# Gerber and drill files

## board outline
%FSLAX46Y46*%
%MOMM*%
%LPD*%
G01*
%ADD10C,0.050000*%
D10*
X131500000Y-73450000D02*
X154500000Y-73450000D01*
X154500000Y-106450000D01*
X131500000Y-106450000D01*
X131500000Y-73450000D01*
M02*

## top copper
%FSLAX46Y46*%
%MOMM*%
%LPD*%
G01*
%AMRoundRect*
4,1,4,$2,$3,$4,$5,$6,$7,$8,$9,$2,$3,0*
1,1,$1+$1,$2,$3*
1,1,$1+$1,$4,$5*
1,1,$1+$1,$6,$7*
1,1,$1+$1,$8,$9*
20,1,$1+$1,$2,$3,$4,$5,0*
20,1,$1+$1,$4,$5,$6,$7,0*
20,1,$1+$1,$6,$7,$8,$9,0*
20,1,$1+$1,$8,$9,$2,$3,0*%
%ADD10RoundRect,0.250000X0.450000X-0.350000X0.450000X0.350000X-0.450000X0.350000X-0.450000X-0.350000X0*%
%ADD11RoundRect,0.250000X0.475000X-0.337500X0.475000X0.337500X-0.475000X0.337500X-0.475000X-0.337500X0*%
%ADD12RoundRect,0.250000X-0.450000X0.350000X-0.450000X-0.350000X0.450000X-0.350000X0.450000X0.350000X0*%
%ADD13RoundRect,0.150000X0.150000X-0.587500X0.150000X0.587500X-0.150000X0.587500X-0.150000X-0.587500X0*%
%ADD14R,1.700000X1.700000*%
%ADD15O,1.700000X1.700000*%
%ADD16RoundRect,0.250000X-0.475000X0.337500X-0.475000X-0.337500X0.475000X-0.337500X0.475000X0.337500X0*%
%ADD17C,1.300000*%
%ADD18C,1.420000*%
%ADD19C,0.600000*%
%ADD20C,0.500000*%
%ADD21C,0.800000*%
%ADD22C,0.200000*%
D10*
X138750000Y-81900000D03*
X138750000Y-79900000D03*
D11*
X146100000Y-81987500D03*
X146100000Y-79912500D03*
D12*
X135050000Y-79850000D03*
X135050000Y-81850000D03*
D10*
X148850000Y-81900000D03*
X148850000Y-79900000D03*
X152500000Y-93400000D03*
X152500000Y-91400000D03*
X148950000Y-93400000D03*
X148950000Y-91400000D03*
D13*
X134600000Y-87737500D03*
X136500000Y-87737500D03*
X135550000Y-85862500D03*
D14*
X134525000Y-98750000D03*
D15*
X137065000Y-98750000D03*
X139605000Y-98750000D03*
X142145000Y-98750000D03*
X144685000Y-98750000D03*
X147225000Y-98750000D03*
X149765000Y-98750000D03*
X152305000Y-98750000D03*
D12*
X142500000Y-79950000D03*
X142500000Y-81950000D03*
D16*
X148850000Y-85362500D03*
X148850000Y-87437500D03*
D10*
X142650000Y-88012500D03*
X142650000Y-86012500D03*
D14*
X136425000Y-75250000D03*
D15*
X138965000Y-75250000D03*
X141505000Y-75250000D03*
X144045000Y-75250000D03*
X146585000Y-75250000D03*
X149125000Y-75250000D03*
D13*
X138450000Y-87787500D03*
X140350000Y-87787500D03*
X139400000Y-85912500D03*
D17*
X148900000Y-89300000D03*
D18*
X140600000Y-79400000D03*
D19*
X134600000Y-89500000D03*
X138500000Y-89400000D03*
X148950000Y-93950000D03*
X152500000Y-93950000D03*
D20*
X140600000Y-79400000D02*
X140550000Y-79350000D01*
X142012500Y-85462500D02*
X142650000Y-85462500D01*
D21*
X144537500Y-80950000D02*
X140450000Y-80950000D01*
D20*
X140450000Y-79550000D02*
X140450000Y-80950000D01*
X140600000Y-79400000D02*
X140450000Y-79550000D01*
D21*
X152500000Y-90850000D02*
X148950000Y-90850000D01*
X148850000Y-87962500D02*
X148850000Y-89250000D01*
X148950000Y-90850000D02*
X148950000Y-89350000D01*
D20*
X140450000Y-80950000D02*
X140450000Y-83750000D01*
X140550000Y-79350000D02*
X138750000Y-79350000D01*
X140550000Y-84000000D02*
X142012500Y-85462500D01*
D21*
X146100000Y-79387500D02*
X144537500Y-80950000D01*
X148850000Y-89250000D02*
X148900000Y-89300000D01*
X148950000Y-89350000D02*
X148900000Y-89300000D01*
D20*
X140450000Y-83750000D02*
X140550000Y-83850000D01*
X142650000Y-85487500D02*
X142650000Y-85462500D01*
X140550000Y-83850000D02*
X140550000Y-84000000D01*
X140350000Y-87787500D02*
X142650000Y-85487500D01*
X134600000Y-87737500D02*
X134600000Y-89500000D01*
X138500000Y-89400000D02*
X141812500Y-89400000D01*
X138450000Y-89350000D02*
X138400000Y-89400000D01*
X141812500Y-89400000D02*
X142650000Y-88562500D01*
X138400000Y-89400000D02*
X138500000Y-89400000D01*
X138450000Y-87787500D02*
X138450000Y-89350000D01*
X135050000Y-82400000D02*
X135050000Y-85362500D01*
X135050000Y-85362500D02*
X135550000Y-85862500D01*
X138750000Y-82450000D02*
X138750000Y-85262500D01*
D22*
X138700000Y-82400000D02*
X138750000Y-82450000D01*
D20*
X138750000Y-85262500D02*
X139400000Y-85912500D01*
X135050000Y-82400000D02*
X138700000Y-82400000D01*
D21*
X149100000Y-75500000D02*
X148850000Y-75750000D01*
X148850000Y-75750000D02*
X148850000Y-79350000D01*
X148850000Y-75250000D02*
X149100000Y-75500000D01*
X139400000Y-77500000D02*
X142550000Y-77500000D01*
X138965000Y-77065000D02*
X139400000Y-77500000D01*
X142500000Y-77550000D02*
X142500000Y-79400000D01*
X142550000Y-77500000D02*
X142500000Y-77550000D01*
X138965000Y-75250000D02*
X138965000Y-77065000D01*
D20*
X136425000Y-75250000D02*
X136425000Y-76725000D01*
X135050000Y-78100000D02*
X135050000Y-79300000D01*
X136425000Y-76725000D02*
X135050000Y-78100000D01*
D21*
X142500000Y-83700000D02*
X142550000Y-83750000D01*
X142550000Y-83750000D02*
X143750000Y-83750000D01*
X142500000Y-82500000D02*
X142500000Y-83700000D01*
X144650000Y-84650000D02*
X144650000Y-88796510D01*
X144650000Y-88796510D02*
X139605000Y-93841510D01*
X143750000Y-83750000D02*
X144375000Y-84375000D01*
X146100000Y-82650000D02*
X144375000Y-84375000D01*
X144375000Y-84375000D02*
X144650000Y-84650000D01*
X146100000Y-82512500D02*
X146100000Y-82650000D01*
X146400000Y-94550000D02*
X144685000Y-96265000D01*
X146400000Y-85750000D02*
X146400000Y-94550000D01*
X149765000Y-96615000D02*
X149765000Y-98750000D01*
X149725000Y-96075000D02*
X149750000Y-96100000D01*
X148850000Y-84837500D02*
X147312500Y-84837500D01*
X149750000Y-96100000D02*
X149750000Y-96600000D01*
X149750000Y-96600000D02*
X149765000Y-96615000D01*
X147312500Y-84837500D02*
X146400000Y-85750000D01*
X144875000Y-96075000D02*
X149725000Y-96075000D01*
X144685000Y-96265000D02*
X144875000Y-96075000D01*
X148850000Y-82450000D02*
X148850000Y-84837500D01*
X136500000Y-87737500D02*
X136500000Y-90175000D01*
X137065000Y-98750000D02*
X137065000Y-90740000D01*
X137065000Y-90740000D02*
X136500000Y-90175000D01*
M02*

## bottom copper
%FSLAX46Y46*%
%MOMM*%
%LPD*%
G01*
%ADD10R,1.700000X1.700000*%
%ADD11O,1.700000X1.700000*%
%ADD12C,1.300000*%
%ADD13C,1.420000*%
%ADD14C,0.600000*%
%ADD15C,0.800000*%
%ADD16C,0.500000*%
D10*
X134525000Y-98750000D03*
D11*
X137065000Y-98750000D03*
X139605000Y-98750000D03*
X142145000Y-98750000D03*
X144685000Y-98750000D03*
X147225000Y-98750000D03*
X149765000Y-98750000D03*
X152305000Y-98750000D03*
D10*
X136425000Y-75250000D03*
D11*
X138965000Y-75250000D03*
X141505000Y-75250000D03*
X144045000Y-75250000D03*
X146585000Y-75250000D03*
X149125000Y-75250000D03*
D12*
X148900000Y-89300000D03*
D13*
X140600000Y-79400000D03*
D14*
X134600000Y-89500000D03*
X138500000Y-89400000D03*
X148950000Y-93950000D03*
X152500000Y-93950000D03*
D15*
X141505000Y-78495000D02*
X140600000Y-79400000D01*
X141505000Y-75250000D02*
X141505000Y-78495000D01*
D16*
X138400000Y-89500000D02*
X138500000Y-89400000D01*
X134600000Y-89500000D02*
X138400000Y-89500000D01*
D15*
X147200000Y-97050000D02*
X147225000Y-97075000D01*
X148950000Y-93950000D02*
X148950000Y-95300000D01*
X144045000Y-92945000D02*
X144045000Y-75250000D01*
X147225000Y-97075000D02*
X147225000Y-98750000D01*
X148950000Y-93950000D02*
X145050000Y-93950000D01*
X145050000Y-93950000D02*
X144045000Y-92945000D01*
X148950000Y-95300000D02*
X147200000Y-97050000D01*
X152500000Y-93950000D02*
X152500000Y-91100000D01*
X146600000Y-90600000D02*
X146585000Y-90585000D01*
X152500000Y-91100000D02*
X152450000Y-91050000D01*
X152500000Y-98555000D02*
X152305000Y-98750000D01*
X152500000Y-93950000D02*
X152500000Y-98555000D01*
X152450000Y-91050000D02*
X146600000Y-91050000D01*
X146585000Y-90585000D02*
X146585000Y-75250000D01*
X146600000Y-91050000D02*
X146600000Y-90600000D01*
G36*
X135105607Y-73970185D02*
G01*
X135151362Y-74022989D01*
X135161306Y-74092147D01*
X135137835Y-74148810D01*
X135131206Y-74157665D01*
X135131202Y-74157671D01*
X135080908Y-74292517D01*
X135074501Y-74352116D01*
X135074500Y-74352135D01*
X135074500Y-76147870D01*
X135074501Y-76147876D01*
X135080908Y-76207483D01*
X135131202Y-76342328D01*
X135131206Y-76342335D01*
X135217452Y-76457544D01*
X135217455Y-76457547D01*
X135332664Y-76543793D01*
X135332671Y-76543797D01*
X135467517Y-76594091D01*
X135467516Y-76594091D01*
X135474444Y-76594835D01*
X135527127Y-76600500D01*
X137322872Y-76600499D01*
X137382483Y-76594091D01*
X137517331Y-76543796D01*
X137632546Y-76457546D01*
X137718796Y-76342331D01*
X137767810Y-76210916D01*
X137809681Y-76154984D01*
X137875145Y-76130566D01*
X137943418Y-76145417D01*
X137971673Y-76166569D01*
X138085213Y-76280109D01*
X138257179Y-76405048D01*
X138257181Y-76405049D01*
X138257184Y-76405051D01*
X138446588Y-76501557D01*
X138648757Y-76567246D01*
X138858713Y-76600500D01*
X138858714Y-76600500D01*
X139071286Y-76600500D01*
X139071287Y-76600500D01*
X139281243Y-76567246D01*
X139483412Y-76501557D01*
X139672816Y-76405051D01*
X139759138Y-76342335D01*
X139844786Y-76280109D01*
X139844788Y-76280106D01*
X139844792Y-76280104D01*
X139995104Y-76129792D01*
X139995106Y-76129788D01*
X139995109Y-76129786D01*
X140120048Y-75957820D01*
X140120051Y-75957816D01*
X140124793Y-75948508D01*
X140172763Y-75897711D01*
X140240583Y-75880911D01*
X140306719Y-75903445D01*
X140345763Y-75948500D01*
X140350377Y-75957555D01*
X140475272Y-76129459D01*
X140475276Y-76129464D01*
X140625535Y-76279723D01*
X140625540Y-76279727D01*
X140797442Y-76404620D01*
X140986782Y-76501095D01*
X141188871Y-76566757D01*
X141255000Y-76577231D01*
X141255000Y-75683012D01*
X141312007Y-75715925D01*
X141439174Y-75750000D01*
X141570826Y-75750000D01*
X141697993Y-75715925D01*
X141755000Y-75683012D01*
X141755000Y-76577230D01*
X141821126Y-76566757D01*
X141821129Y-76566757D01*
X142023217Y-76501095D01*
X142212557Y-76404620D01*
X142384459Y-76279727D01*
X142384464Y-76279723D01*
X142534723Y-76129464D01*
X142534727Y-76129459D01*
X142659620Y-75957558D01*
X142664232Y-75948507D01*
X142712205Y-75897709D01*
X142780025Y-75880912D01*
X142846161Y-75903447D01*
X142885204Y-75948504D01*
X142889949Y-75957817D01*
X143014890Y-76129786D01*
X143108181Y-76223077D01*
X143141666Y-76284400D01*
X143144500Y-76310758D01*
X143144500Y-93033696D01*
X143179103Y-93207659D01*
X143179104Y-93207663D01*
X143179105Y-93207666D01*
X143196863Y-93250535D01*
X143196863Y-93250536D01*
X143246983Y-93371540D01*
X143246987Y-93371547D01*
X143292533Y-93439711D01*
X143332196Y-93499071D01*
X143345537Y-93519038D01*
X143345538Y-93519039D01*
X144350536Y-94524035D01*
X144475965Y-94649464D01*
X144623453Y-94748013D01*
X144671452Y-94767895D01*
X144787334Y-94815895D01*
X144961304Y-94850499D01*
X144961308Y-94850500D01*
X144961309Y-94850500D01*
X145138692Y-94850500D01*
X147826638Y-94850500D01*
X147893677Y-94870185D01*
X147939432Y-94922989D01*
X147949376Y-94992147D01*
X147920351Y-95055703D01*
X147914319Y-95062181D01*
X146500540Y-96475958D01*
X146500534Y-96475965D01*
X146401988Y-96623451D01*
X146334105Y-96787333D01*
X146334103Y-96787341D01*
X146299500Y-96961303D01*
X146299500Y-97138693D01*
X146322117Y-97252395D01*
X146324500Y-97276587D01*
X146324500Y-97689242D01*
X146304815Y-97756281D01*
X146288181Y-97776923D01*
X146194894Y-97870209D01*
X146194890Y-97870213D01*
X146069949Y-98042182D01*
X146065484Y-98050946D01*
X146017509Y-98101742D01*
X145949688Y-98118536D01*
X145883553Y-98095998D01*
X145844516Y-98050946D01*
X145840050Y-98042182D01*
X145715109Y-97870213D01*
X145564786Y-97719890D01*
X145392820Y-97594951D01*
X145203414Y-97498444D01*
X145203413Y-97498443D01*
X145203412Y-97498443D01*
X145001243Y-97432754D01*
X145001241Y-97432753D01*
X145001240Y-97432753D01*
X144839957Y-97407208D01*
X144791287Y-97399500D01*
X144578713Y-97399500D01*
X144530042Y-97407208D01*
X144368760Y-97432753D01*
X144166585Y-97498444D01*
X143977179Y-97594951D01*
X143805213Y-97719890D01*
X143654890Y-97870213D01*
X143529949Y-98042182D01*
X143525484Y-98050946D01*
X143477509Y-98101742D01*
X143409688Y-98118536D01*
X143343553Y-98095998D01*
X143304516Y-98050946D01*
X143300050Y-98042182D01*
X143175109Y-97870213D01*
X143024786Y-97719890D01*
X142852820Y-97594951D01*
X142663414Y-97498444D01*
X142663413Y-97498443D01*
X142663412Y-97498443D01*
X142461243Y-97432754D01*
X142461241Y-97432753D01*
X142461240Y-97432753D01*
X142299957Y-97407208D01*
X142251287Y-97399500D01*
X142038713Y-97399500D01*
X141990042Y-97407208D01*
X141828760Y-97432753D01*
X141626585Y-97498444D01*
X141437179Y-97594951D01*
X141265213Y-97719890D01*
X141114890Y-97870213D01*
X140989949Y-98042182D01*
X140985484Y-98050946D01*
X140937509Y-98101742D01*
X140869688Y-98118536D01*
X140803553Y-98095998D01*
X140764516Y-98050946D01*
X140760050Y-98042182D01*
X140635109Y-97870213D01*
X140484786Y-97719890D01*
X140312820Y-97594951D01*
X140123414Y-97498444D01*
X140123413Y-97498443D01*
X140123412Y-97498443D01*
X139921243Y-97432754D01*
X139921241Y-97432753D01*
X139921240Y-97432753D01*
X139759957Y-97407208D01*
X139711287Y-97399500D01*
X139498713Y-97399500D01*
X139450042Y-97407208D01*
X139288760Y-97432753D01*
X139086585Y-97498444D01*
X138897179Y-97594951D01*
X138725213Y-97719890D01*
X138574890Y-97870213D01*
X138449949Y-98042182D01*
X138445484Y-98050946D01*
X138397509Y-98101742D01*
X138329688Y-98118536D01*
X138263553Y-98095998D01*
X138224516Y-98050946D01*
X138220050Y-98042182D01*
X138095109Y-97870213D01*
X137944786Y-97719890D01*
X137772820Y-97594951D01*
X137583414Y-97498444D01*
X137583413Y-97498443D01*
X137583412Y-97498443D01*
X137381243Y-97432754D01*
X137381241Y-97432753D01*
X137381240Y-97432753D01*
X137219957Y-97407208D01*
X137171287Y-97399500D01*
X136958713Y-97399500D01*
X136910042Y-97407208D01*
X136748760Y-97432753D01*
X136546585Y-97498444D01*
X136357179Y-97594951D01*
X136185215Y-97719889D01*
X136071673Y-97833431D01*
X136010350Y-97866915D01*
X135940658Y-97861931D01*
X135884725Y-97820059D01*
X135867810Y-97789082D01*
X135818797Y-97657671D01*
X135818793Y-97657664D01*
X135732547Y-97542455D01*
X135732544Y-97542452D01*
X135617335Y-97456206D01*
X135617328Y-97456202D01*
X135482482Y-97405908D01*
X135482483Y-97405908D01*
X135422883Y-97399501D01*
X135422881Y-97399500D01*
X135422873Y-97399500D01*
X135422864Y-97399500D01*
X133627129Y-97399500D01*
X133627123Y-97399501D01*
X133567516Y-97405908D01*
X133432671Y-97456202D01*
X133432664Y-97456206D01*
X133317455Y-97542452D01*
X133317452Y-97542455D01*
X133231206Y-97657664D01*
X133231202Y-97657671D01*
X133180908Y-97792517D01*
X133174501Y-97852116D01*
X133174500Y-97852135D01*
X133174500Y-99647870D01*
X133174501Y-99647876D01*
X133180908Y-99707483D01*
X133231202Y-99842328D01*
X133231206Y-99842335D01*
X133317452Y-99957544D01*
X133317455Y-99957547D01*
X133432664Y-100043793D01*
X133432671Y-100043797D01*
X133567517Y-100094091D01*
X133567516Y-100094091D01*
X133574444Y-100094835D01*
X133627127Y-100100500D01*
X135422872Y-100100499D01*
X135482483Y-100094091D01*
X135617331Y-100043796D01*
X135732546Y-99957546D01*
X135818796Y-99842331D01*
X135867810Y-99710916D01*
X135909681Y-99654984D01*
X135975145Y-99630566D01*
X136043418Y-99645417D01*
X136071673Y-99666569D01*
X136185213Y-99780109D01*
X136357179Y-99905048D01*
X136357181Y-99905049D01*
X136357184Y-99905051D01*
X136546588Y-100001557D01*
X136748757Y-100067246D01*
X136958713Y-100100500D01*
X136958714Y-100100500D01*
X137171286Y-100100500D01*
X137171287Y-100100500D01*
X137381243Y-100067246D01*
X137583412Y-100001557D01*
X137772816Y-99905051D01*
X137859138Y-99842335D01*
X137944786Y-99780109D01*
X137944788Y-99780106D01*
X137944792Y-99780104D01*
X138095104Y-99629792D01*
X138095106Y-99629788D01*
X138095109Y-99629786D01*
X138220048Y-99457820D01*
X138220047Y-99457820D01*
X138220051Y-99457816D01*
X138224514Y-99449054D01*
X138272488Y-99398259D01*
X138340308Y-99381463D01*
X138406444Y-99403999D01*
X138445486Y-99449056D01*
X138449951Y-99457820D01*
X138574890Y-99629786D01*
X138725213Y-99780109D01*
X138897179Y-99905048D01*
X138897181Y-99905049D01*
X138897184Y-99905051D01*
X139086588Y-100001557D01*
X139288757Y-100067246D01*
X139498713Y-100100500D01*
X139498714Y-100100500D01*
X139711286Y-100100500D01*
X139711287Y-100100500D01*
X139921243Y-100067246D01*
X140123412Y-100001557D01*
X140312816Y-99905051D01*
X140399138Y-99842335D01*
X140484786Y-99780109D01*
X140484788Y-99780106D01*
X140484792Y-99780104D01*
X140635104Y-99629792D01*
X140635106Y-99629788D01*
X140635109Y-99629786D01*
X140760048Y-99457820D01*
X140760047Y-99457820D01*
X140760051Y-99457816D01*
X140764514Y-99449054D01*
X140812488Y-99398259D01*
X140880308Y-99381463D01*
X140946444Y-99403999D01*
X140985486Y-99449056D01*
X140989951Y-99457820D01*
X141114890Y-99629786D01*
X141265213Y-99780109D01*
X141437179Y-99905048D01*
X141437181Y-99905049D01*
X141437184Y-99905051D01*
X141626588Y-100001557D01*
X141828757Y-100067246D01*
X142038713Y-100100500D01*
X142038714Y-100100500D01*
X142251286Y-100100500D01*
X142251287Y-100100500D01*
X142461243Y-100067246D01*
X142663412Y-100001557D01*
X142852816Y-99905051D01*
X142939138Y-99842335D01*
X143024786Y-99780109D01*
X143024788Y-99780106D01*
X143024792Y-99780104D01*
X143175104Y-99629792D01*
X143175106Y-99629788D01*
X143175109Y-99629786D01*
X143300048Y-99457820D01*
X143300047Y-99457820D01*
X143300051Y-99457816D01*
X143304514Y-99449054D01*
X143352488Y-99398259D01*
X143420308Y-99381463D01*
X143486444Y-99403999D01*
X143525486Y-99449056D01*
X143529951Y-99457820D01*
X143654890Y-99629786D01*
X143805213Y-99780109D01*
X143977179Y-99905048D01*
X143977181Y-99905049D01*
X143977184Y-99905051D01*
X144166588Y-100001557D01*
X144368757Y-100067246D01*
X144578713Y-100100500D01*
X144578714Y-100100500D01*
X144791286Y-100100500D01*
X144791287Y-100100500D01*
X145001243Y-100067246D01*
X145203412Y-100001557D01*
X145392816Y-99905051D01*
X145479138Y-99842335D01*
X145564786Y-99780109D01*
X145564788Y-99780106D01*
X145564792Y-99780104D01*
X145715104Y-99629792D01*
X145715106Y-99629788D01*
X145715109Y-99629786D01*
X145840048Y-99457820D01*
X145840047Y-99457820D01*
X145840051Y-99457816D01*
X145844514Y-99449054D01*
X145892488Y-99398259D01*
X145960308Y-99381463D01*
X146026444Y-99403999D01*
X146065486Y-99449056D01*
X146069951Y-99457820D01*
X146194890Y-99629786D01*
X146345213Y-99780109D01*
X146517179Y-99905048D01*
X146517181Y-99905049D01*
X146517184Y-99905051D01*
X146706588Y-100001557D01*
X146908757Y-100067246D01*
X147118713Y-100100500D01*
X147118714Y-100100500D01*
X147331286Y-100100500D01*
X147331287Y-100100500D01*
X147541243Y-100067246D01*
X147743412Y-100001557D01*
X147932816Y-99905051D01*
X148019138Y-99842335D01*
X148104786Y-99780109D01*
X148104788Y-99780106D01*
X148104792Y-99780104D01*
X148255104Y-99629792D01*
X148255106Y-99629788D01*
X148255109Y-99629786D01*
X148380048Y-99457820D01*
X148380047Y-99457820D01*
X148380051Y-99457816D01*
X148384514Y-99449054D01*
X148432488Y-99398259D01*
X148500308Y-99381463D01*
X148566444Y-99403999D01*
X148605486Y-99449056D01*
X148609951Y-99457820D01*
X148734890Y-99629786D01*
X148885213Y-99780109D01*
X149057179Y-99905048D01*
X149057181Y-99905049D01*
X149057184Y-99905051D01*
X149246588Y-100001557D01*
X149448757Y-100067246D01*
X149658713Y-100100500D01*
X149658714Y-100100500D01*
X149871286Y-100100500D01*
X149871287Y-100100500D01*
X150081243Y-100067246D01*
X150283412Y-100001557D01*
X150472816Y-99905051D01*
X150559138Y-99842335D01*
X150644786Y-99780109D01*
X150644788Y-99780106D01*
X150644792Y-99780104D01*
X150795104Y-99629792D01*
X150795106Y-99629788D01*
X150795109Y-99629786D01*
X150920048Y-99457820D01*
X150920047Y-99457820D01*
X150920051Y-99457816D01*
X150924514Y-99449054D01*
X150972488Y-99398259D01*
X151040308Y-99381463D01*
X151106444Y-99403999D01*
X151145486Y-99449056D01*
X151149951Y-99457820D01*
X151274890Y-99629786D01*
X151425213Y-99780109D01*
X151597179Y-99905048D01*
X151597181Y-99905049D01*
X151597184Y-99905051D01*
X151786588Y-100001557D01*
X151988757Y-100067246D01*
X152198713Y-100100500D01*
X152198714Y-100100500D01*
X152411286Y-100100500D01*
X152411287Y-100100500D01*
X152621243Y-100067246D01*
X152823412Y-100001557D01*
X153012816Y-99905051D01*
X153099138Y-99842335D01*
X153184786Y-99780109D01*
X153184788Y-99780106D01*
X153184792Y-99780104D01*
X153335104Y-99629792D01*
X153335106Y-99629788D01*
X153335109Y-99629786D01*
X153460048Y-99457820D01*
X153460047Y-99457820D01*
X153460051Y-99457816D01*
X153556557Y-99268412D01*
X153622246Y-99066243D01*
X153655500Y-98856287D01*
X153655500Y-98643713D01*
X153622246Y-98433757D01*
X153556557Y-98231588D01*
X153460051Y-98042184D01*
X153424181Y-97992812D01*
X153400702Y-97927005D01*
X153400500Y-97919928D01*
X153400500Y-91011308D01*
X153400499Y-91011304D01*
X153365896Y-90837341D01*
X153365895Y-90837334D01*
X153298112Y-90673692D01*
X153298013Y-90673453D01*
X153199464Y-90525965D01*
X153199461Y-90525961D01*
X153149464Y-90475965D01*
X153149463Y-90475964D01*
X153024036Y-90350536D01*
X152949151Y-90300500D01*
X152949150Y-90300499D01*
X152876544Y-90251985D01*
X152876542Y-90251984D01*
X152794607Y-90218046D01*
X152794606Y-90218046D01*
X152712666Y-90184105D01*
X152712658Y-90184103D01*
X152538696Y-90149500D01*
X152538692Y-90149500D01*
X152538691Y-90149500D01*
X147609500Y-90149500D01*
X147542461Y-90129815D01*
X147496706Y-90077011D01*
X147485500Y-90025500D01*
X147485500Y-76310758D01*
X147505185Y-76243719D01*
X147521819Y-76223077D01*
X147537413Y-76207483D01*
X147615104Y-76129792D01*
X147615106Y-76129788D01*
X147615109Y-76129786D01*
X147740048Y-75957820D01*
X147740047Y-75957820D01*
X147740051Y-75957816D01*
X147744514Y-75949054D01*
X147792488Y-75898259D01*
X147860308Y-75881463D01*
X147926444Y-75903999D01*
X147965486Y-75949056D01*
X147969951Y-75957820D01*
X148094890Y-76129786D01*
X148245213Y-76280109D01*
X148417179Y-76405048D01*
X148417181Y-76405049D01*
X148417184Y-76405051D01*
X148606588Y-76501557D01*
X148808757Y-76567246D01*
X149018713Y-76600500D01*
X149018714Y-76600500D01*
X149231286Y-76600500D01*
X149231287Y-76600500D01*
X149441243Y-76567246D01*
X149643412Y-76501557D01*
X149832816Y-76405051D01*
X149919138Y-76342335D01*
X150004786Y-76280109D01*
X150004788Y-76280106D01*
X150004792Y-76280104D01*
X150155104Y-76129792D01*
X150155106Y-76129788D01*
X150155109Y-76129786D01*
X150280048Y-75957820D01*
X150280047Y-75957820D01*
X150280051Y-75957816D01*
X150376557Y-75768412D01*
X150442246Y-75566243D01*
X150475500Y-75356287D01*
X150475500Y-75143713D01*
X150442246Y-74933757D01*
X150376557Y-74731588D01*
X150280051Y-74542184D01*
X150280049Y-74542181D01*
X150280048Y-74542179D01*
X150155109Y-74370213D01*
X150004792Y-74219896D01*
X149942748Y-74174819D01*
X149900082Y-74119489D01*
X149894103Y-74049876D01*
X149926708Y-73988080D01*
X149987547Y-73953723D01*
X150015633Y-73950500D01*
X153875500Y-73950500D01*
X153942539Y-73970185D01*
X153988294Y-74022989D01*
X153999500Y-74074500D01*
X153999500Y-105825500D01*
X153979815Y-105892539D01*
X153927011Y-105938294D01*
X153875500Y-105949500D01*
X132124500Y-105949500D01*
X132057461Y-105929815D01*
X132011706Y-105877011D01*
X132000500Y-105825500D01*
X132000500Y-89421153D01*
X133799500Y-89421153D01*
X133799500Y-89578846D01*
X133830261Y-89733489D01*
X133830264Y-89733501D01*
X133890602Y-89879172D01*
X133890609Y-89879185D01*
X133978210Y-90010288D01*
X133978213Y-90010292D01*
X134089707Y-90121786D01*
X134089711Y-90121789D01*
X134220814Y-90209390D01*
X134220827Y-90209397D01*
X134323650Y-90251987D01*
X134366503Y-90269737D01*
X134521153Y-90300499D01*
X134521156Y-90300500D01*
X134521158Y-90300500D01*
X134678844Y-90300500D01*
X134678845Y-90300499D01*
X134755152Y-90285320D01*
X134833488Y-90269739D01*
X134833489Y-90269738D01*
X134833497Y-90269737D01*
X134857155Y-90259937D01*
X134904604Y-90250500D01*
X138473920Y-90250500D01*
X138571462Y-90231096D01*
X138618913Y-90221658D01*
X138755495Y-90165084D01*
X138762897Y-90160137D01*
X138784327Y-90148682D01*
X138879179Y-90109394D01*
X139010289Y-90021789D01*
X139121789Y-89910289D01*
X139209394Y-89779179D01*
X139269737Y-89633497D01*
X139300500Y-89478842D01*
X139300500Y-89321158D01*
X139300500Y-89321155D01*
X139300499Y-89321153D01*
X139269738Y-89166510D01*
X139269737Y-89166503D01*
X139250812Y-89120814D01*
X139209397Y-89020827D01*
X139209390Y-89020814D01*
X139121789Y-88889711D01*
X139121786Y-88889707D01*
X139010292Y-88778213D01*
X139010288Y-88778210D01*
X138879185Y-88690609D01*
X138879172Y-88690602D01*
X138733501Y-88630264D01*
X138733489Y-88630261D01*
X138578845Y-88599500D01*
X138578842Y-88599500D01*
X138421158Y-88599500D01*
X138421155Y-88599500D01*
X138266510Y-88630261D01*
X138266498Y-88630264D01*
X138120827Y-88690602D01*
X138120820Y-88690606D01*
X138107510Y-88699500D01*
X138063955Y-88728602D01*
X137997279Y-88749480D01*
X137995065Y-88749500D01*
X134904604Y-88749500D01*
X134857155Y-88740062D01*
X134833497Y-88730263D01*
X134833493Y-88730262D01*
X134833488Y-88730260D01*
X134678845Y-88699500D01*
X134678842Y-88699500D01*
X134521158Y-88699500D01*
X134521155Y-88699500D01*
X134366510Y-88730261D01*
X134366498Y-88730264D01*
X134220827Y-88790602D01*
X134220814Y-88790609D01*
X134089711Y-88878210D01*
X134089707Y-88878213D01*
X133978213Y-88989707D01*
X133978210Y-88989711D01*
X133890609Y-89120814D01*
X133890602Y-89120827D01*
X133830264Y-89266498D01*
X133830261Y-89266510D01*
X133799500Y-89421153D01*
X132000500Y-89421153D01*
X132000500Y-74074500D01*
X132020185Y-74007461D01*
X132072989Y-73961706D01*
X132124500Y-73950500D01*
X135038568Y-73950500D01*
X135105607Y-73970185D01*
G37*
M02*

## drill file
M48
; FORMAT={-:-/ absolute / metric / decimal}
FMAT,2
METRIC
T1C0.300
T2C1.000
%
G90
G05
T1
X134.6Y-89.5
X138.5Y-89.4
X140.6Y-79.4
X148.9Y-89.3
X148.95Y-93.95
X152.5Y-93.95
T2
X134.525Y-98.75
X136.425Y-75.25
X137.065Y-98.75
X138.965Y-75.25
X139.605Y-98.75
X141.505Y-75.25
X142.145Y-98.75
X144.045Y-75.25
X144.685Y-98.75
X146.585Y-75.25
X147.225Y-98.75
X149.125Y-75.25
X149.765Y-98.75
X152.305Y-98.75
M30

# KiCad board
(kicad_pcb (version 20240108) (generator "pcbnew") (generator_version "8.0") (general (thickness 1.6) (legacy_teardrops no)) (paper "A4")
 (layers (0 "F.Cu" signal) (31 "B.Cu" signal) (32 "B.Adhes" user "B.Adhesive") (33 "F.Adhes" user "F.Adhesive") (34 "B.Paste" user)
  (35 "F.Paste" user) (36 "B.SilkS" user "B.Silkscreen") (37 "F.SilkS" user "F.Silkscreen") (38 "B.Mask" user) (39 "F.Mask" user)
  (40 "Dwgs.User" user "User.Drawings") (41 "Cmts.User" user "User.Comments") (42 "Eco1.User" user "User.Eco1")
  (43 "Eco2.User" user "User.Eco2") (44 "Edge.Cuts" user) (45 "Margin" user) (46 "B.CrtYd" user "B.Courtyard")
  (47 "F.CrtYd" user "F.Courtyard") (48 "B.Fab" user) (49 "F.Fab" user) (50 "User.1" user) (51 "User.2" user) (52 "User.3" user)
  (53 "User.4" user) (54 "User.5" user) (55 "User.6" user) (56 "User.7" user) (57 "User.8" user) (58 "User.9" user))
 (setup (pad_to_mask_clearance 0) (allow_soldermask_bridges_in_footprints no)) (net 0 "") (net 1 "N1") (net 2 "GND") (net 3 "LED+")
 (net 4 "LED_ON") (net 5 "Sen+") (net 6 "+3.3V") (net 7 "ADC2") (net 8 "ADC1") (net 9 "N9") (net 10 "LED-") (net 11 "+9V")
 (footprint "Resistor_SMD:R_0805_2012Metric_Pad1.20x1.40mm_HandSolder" (layer "F.Cu") (at 138.75 80.9 90)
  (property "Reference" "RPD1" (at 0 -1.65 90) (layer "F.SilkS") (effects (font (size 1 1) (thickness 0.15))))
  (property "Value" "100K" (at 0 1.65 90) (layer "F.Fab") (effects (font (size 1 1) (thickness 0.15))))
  (pad "1" smd roundrect (at -1 0 90) (size 1.2 1.4) (layers "F.Cu" "F.Paste" "F.Mask") (roundrect_rratio 0.208333) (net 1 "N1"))
  (pad "2" smd roundrect (at 1 0 90) (size 1.2 1.4) (layers "F.Cu" "F.Paste" "F.Mask") (roundrect_rratio 0.208333) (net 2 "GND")))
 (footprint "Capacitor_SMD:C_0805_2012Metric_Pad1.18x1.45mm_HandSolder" (layer "F.Cu") (at 146.1 80.95 90)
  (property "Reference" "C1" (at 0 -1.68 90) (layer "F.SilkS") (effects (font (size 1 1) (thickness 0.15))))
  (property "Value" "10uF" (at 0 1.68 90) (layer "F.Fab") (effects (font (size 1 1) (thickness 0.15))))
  (pad "1" smd roundrect (at -1.0375 0 90) (size 1.175 1.45) (layers "F.Cu" "F.Paste" "F.Mask") (roundrect_rratio 0.212766) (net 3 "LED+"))
  (pad "2" smd roundrect (at 1.0375 0 90) (size 1.175 1.45) (layers "F.Cu" "F.Paste" "F.Mask") (roundrect_rratio 0.212766) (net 2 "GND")))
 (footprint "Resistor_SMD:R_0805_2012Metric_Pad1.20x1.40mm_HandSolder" (layer "F.Cu") (at 135.05 80.85 -90)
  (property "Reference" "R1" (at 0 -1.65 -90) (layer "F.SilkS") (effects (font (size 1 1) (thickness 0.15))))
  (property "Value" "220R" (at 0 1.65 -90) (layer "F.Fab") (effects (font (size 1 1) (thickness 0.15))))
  (pad "1" smd roundrect (at -1 0 270) (size 1.2 1.4) (layers "F.Cu" "F.Paste" "F.Mask") (roundrect_rratio 0.208333) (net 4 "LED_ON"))
  (pad "2" smd roundrect (at 1 0 270) (size 1.2 1.4) (layers "F.Cu" "F.Paste" "F.Mask") (roundrect_rratio 0.208333) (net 1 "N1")))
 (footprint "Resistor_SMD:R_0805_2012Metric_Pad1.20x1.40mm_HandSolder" (layer "F.Cu") (at 148.85 80.9 90)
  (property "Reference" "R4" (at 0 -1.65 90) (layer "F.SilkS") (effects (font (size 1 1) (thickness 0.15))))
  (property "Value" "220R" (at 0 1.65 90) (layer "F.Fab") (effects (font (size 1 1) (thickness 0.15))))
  (pad "1" smd roundrect (at -1 0 90) (size 1.2 1.4) (layers "F.Cu" "F.Paste" "F.Mask") (roundrect_rratio 0.208333) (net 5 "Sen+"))
  (pad "2" smd roundrect (at 1 0 90) (size 1.2 1.4) (layers "F.Cu" "F.Paste" "F.Mask") (roundrect_rratio 0.208333) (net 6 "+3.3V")))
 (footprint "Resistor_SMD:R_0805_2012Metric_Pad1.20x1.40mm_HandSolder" (layer "F.Cu") (at 152.5 92.4 90)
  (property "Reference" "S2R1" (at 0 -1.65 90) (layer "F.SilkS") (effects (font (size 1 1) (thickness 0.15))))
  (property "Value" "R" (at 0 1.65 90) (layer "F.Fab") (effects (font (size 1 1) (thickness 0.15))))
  (pad "1" smd roundrect (at -1 0 90) (size 1.2 1.4) (layers "F.Cu" "F.Paste" "F.Mask") (roundrect_rratio 0.208333) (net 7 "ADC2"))
  (pad "2" smd roundrect (at 1 0 90) (size 1.2 1.4) (layers "F.Cu" "F.Paste" "F.Mask") (roundrect_rratio 0.208333) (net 2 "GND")))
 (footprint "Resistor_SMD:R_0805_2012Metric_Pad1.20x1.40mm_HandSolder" (layer "F.Cu") (at 148.95 92.4 90)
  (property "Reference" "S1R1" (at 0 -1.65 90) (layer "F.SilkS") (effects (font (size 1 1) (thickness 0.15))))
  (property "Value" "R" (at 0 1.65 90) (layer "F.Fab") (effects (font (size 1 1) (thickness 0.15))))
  (pad "1" smd roundrect (at -1 0 90) (size 1.2 1.4) (layers "F.Cu" "F.Paste" "F.Mask") (roundrect_rratio 0.208333) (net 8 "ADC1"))
  (pad "2" smd roundrect (at 1 0 90) (size 1.2 1.4) (layers "F.Cu" "F.Paste" "F.Mask") (roundrect_rratio 0.208333) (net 2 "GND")))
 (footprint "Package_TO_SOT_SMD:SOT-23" (layer "F.Cu") (at 135.55 86.8 90)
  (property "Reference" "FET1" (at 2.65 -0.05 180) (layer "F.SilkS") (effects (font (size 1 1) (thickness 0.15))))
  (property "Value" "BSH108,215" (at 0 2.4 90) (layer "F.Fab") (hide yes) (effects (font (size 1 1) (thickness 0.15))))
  (pad "1" smd roundrect (at -0.9375 -0.95 90) (size 1.475 0.6) (layers "F.Cu" "F.Paste" "F.Mask") (roundrect_rratio 0.25) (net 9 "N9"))
  (pad "2" smd roundrect (at -0.9375 0.95 90) (size 1.475 0.6) (layers "F.Cu" "F.Paste" "F.Mask") (roundrect_rratio 0.25) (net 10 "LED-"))
  (pad "3" smd roundrect (at 0.9375 0 90) (size 1.475 0.6) (layers "F.Cu" "F.Paste" "F.Mask") (roundrect_rratio 0.25) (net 1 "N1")))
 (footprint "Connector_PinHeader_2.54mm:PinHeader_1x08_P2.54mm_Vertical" (layer "F.Cu") (at 134.525 98.75 90)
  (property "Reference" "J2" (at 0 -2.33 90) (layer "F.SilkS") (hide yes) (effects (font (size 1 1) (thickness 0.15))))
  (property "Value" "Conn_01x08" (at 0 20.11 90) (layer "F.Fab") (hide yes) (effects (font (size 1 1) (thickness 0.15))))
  (pad "1" thru_hole rect (at 0 0 90) (size 1.7 1.7) (drill 1) (layers "*.Cu" "*.Mask") (remove_unused_layers no) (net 3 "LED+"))
  (pad "2" thru_hole oval (at 0 2.54 90) (size 1.7 1.7) (drill 1) (layers "*.Cu" "*.Mask") (remove_unused_layers no) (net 10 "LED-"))
  (pad "3" thru_hole oval (at 0 5.08 90) (size 1.7 1.7) (drill 1) (layers "*.Cu" "*.Mask") (remove_unused_layers no) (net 5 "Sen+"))
  (pad "4" thru_hole oval (at 0 7.62 90) (size 1.7 1.7) (drill 1) (layers "*.Cu" "*.Mask") (remove_unused_layers no) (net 8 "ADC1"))
  (pad "5" thru_hole oval (at 0 10.16 90) (size 1.7 1.7) (drill 1) (layers "*.Cu" "*.Mask") (remove_unused_layers no) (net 3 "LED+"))
  (pad "6" thru_hole oval (at 0 12.7 90) (size 1.7 1.7) (drill 1) (layers "*.Cu" "*.Mask") (remove_unused_layers no) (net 10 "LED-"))
  (pad "7" thru_hole oval (at 0 15.24 90) (size 1.7 1.7) (drill 1) (layers "*.Cu" "*.Mask") (remove_unused_layers no) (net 5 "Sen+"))
  (pad "8" thru_hole oval (at 0 17.78 90) (size 1.7 1.7) (drill 1) (layers "*.Cu" "*.Mask") (remove_unused_layers no) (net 7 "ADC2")))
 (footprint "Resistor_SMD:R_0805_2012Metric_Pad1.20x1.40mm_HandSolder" (layer "F.Cu") (at 142.5 80.95 -90)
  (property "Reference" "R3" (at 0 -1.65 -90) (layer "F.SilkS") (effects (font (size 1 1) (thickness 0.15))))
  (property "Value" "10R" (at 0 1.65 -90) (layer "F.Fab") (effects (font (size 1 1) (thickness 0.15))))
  (pad "1" smd roundrect (at -1 0 270) (size 1.2 1.4) (layers "F.Cu" "F.Paste" "F.Mask") (roundrect_rratio 0.208333) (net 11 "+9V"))
  (pad "2" smd roundrect (at 1 0 270) (size 1.2 1.4) (layers "F.Cu" "F.Paste" "F.Mask") (roundrect_rratio 0.208333) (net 3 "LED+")))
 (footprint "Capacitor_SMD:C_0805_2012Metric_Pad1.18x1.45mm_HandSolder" (layer "F.Cu") (at 148.85 86.4 -90)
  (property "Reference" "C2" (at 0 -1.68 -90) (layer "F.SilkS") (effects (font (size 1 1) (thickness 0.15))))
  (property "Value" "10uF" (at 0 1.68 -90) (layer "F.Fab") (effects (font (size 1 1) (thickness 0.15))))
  (pad "1" smd roundrect (at -1.0375 0 270) (size 1.175 1.45) (layers "F.Cu" "F.Paste" "F.Mask") (roundrect_rratio 0.212766) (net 5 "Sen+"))
  (pad "2" smd roundrect (at 1.0375 0 270) (size 1.175 1.45) (layers "F.Cu" "F.Paste" "F.Mask") (roundrect_rratio 0.212766) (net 2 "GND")))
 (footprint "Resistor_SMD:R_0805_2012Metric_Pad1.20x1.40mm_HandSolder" (layer "F.Cu") (at 142.65 87.0125 90)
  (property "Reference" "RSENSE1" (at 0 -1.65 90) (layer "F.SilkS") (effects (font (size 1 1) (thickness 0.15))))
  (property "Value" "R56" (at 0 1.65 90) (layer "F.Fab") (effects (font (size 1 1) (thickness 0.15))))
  (pad "1" smd roundrect (at -1 0 90) (size 1.2 1.4) (layers "F.Cu" "F.Paste" "F.Mask") (roundrect_rratio 0.208333) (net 9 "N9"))
  (pad "2" smd roundrect (at 1 0 90) (size 1.2 1.4) (layers "F.Cu" "F.Paste" "F.Mask") (roundrect_rratio 0.208333) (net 2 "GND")))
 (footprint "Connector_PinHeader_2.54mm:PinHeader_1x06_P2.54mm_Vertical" (layer "F.Cu") (at 136.425 75.25 90)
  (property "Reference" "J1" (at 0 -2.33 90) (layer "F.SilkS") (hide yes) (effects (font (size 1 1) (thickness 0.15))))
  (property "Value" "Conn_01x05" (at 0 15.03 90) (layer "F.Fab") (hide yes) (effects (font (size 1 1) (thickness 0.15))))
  (pad "1" thru_hole rect (at 0 0 90) (size 1.7 1.7) (drill 1) (layers "*.Cu" "*.Mask") (remove_unused_layers no) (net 4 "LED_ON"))
  (pad "2" thru_hole oval (at 0 2.54 90) (size 1.7 1.7) (drill 1) (layers "*.Cu" "*.Mask") (remove_unused_layers no) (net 11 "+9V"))
  (pad "3" thru_hole oval (at 0 5.08 90) (size 1.7 1.7) (drill 1) (layers "*.Cu" "*.Mask") (remove_unused_layers no) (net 2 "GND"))
  (pad "4" thru_hole oval (at 0 7.62 90) (size 1.7 1.7) (drill 1) (layers "*.Cu" "*.Mask") (remove_unused_layers no) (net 8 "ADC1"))
  (pad "5" thru_hole oval (at 0 10.16 90) (size 1.7 1.7) (drill 1) (layers "*.Cu" "*.Mask") (remove_unused_layers no) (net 7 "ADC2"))
  (pad "6" thru_hole oval (at 0 12.7 90) (size 1.7 1.7) (drill 1) (layers "*.Cu" "*.Mask") (remove_unused_layers no) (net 6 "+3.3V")))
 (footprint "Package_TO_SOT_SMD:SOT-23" (layer "F.Cu") (at 139.4 86.85 90)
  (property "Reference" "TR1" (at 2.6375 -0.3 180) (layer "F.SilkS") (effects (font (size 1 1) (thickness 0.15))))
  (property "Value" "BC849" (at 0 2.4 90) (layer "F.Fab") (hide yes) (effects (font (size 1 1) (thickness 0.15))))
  (pad "1" smd roundrect (at -0.9375 -0.95 90) (size 1.475 0.6) (layers "F.Cu" "F.Paste" "F.Mask") (roundrect_rratio 0.25) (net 9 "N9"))
  (pad "2" smd roundrect (at -0.9375 0.95 90) (size 1.475 0.6) (layers "F.Cu" "F.Paste" "F.Mask") (roundrect_rratio 0.25) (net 2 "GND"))
  (pad "3" smd roundrect (at 0.9375 0 90) (size 1.475 0.6) (layers "F.Cu" "F.Paste" "F.Mask") (roundrect_rratio 0.25) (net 1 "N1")))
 (gr_rect (start 131.5 73.45) (end 154.5 106.45) (stroke (width 0.05) (type default)) (fill none) (layer "Edge.Cuts"))
 (segment (start 140.6 79.4) (end 140.55 79.35) (width 0.5) (layer "F.Cu") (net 2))
 (segment (start 142.0125 85.4625) (end 142.65 85.4625) (width 0.5) (layer "F.Cu") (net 2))
 (segment (start 144.5375 80.95) (end 140.45 80.95) (width 0.8) (layer "F.Cu") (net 2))
 (segment (start 140.45 79.55) (end 140.45 80.95) (width 0.5) (layer "F.Cu") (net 2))
 (segment (start 140.6 79.4) (end 140.45 79.55) (width 0.5) (layer "F.Cu") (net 2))
 (segment (start 152.5 90.85) (end 148.95 90.85) (width 0.8) (layer "F.Cu") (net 2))
 (segment (start 148.85 87.9625) (end 148.85 89.25) (width 0.8) (layer "F.Cu") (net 2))
 (segment (start 148.95 90.85) (end 148.95 89.35) (width 0.8) (layer "F.Cu") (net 2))
 (segment (start 140.45 80.95) (end 140.45 83.75) (width 0.5) (layer "F.Cu") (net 2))
 (segment (start 140.55 79.35) (end 138.75 79.35) (width 0.5) (layer "F.Cu") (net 2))
 (segment (start 140.55 84) (end 142.0125 85.4625) (width 0.5) (layer "F.Cu") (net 2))
 (segment (start 146.1 79.3875) (end 144.5375 80.95) (width 0.8) (layer "F.Cu") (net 2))
 (segment (start 148.85 89.25) (end 148.9 89.3) (width 0.8) (layer "F.Cu") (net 2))
 (segment (start 148.95 89.35) (end 148.9 89.3) (width 0.8) (layer "F.Cu") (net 2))
 (segment (start 140.45 83.75) (end 140.55 83.85) (width 0.5) (layer "F.Cu") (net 2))
 (segment (start 142.65 85.4875) (end 142.65 85.4625) (width 0.5) (layer "F.Cu") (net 2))
 (segment (start 140.55 83.85) (end 140.55 84) (width 0.5) (layer "F.Cu") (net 2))
 (segment (start 140.35 87.7875) (end 142.65 85.4875) (width 0.5) (layer "F.Cu") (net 2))
 (via (at 148.9 89.3) (size 1.3) (drill 0.3) (layers "F.Cu" "B.Cu") (free yes) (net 2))
 (via (at 140.6 79.4) (size 1.42) (drill 0.3) (layers "F.Cu" "B.Cu") (free yes) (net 2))
 (segment (start 141.505 78.495) (end 140.6 79.4) (width 0.8) (layer "B.Cu") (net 2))
 (segment (start 141.505 75.25) (end 141.505 78.495) (width 0.8) (layer "B.Cu") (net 2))
 (segment (start 134.6 87.7375) (end 134.6 89.5) (width 0.5) (layer "F.Cu") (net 9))
 (segment (start 138.5 89.4) (end 141.8125 89.4) (width 0.5) (layer "F.Cu") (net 9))
 (segment (start 138.45 89.35) (end 138.4 89.4) (width 0.5) (layer "F.Cu") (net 9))
 (segment (start 141.8125 89.4) (end 142.65 88.5625) (width 0.5) (layer "F.Cu") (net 9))
 (segment (start 138.4 89.4) (end 138.5 89.4) (width 0.5) (layer "F.Cu") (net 9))
 (segment (start 138.45 87.7875) (end 138.45 89.35) (width 0.5) (layer "F.Cu") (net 9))
 (via (at 134.6 89.5) (size 0.6) (drill 0.3) (layers "F.Cu" "B.Cu") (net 9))
 (via (at 138.5 89.4) (size 0.6) (drill 0.3) (layers "F.Cu" "B.Cu") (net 9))
 (segment (start 138.4 89.5) (end 138.5 89.4) (width 0.5) (layer "B.Cu") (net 9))
 (segment (start 134.6 89.5) (end 138.4 89.5) (width 0.5) (layer "B.Cu") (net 9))
 (segment (start 135.05 82.4) (end 135.05 85.3625) (width 0.5) (layer "F.Cu") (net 1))
 (segment (start 135.05 85.3625) (end 135.55 85.8625) (width 0.5) (layer "F.Cu") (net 1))
 (segment (start 138.75 82.45) (end 138.75 85.2625) (width 0.5) (layer "F.Cu") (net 1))
 (segment (start 138.7 82.4) (end 138.75 82.45) (width 0.2) (layer "F.Cu") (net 1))
 (segment (start 138.75 85.2625) (end 139.4 85.9125) (width 0.5) (layer "F.Cu") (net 1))
 (segment (start 135.05 82.4) (end 138.7 82.4) (width 0.5) (layer "F.Cu") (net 1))
 (segment (start 149.1 75.5) (end 148.85 75.75) (width 0.8) (layer "F.Cu") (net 6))
 (segment (start 148.85 75.75) (end 148.85 79.35) (width 0.8) (layer "F.Cu") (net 6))
 (segment (start 148.85 75.25) (end 149.1 75.5) (width 0.8) (layer "F.Cu") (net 6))
 (segment (start 139.4 77.5) (end 142.55 77.5) (width 0.8) (layer "F.Cu") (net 11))
 (segment (start 138.965 77.065) (end 139.4 77.5) (width 0.8) (layer "F.Cu") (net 11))
 (segment (start 142.5 77.55) (end 142.5 79.4) (width 0.8) (layer "F.Cu") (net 11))
 (segment (start 142.55 77.5) (end 142.5 77.55) (width 0.8) (layer "F.Cu") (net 11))
 (segment (start 138.965 75.25) (end 138.965 77.065) (width 0.8) (layer "F.Cu") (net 11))
 (via (at 148.95 93.95) (size 0.6) (drill 0.3) (layers "F.Cu" "B.Cu") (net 8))
 (segment (start 147.2 97.05) (end 147.225 97.075) (width 0.8) (layer "B.Cu") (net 8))
 (segment (start 148.95 93.95) (end 148.95 95.3) (width 0.8) (layer "B.Cu") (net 8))
 (segment (start 144.045 92.945) (end 144.045 75.25) (width 0.8) (layer "B.Cu") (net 8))
 (segment (start 147.225 97.075) (end 147.225 98.75) (width 0.8) (layer "B.Cu") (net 8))
 (segment (start 148.95 93.95) (end 145.05 93.95) (width 0.8) (layer "B.Cu") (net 8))
 (segment (start 145.05 93.95) (end 144.045 92.945) (width 0.8) (layer "B.Cu") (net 8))
 (segment (start 148.95 95.3) (end 147.2 97.05) (width 0.8) (layer "B.Cu") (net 8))
 (segment (start 136.425 75.25) (end 136.425 76.725) (width 0.5) (layer "F.Cu") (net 4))
 (segment (start 135.05 78.1) (end 135.05 79.3) (width 0.5) (layer "F.Cu") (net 4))
 (segment (start 136.425 76.725) (end 135.05 78.1) (width 0.5) (layer "F.Cu") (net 4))
 (segment (start 142.5 83.7) (end 142.55 83.75) (width 0.8) (layer "F.Cu") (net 3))
 (segment (start 142.55 83.75) (end 143.75 83.75) (width 0.8) (layer "F.Cu") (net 3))
 (segment (start 142.5 82.5) (end 142.5 83.7) (width 0.8) (layer "F.Cu") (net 3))
 (segment (start 144.65 84.65) (end 144.65 88.79651) (width 0.8) (layer "F.Cu") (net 3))
 (segment (start 144.65 88.79651) (end 139.605 93.84151) (width 0.8) (layer "F.Cu") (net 3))
 (segment (start 143.75 83.75) (end 144.375 84.375) (width 0.8) (layer "F.Cu") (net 3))
 (segment (start 146.1 82.65) (end 144.375 84.375) (width 0.8) (layer "F.Cu") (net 3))
 (segment (start 144.375 84.375) (end 144.65 84.65) (width 0.8) (layer "F.Cu") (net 3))
 (segment (start 146.1 82.5125) (end 146.1 82.65) (width 0.8) (layer "F.Cu") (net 3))
 (segment (start 146.4 94.55) (end 144.685 96.265) (width 0.8) (layer "F.Cu") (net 5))
 (segment (start 146.4 85.75) (end 146.4 94.55) (width 0.8) (layer "F.Cu") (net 5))
 (segment (start 149.765 96.615) (end 149.765 98.75) (width 0.8) (layer "F.Cu") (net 5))
 (segment (start 149.725 96.075) (end 149.75 96.1) (width 0.8) (layer "F.Cu") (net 5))
 (segment (start 148.85 84.8375) (end 147.3125 84.8375) (width 0.8) (layer "F.Cu") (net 5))
 (segment (start 149.75 96.1) (end 149.75 96.6) (width 0.8) (layer "F.Cu") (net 5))
 (segment (start 149.75 96.6) (end 149.765 96.615) (width 0.8) (layer "F.Cu") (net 5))
 (segment (start 147.3125 84.8375) (end 146.4 85.75) (width 0.8) (layer "F.Cu") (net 5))
 (segment (start 144.875 96.075) (end 149.725 96.075) (width 0.8) (layer "F.Cu") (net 5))
 (segment (start 144.685 96.265) (end 144.875 96.075) (width 0.8) (layer "F.Cu") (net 5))
 (segment (start 148.85 82.45) (end 148.85 84.8375) (width 0.8) (layer "F.Cu") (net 5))
 (segment (start 136.5 87.7375) (end 136.5 90.175) (width 0.8) (layer "F.Cu") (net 10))
 (segment (start 137.065 98.75) (end 137.065 90.74) (width 0.8) (layer "F.Cu") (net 10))
 (segment (start 137.065 90.74) (end 136.5 90.175) (width 0.8) (layer "F.Cu") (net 10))
 (via (at 152.5 93.95) (size 0.6) (drill 0.3) (layers "F.Cu" "B.Cu") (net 7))
 (segment (start 152.5 93.95) (end 152.5 91.1) (width 0.8) (layer "B.Cu") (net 7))
 (segment (start 146.6 90.6) (end 146.585 90.585) (width 0.8) (layer "B.Cu") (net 7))
 (segment (start 152.5 91.1) (end 152.45 91.05) (width 0.8) (layer "B.Cu") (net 7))
 (segment (start 152.5 98.555) (end 152.305 98.75) (width 0.8) (layer "B.Cu") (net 7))
 (segment (start 152.5 93.95) (end 152.5 98.555) (width 0.8) (layer "B.Cu") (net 7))
 (segment (start 152.45 91.05) (end 146.6 91.05) (width 0.8) (layer "B.Cu") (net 7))
 (segment (start 146.585 90.585) (end 146.585 75.25) (width 0.8) (layer "B.Cu") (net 7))
 (segment (start 146.6 91.05) (end 146.6 90.6) (width 0.8) (layer "B.Cu") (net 7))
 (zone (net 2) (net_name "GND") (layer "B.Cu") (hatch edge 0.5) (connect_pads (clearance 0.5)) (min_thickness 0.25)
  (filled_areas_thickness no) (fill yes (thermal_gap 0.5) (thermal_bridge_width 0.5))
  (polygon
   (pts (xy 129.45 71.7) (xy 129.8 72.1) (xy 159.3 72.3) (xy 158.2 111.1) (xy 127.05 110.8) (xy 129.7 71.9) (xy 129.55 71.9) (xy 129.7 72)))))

